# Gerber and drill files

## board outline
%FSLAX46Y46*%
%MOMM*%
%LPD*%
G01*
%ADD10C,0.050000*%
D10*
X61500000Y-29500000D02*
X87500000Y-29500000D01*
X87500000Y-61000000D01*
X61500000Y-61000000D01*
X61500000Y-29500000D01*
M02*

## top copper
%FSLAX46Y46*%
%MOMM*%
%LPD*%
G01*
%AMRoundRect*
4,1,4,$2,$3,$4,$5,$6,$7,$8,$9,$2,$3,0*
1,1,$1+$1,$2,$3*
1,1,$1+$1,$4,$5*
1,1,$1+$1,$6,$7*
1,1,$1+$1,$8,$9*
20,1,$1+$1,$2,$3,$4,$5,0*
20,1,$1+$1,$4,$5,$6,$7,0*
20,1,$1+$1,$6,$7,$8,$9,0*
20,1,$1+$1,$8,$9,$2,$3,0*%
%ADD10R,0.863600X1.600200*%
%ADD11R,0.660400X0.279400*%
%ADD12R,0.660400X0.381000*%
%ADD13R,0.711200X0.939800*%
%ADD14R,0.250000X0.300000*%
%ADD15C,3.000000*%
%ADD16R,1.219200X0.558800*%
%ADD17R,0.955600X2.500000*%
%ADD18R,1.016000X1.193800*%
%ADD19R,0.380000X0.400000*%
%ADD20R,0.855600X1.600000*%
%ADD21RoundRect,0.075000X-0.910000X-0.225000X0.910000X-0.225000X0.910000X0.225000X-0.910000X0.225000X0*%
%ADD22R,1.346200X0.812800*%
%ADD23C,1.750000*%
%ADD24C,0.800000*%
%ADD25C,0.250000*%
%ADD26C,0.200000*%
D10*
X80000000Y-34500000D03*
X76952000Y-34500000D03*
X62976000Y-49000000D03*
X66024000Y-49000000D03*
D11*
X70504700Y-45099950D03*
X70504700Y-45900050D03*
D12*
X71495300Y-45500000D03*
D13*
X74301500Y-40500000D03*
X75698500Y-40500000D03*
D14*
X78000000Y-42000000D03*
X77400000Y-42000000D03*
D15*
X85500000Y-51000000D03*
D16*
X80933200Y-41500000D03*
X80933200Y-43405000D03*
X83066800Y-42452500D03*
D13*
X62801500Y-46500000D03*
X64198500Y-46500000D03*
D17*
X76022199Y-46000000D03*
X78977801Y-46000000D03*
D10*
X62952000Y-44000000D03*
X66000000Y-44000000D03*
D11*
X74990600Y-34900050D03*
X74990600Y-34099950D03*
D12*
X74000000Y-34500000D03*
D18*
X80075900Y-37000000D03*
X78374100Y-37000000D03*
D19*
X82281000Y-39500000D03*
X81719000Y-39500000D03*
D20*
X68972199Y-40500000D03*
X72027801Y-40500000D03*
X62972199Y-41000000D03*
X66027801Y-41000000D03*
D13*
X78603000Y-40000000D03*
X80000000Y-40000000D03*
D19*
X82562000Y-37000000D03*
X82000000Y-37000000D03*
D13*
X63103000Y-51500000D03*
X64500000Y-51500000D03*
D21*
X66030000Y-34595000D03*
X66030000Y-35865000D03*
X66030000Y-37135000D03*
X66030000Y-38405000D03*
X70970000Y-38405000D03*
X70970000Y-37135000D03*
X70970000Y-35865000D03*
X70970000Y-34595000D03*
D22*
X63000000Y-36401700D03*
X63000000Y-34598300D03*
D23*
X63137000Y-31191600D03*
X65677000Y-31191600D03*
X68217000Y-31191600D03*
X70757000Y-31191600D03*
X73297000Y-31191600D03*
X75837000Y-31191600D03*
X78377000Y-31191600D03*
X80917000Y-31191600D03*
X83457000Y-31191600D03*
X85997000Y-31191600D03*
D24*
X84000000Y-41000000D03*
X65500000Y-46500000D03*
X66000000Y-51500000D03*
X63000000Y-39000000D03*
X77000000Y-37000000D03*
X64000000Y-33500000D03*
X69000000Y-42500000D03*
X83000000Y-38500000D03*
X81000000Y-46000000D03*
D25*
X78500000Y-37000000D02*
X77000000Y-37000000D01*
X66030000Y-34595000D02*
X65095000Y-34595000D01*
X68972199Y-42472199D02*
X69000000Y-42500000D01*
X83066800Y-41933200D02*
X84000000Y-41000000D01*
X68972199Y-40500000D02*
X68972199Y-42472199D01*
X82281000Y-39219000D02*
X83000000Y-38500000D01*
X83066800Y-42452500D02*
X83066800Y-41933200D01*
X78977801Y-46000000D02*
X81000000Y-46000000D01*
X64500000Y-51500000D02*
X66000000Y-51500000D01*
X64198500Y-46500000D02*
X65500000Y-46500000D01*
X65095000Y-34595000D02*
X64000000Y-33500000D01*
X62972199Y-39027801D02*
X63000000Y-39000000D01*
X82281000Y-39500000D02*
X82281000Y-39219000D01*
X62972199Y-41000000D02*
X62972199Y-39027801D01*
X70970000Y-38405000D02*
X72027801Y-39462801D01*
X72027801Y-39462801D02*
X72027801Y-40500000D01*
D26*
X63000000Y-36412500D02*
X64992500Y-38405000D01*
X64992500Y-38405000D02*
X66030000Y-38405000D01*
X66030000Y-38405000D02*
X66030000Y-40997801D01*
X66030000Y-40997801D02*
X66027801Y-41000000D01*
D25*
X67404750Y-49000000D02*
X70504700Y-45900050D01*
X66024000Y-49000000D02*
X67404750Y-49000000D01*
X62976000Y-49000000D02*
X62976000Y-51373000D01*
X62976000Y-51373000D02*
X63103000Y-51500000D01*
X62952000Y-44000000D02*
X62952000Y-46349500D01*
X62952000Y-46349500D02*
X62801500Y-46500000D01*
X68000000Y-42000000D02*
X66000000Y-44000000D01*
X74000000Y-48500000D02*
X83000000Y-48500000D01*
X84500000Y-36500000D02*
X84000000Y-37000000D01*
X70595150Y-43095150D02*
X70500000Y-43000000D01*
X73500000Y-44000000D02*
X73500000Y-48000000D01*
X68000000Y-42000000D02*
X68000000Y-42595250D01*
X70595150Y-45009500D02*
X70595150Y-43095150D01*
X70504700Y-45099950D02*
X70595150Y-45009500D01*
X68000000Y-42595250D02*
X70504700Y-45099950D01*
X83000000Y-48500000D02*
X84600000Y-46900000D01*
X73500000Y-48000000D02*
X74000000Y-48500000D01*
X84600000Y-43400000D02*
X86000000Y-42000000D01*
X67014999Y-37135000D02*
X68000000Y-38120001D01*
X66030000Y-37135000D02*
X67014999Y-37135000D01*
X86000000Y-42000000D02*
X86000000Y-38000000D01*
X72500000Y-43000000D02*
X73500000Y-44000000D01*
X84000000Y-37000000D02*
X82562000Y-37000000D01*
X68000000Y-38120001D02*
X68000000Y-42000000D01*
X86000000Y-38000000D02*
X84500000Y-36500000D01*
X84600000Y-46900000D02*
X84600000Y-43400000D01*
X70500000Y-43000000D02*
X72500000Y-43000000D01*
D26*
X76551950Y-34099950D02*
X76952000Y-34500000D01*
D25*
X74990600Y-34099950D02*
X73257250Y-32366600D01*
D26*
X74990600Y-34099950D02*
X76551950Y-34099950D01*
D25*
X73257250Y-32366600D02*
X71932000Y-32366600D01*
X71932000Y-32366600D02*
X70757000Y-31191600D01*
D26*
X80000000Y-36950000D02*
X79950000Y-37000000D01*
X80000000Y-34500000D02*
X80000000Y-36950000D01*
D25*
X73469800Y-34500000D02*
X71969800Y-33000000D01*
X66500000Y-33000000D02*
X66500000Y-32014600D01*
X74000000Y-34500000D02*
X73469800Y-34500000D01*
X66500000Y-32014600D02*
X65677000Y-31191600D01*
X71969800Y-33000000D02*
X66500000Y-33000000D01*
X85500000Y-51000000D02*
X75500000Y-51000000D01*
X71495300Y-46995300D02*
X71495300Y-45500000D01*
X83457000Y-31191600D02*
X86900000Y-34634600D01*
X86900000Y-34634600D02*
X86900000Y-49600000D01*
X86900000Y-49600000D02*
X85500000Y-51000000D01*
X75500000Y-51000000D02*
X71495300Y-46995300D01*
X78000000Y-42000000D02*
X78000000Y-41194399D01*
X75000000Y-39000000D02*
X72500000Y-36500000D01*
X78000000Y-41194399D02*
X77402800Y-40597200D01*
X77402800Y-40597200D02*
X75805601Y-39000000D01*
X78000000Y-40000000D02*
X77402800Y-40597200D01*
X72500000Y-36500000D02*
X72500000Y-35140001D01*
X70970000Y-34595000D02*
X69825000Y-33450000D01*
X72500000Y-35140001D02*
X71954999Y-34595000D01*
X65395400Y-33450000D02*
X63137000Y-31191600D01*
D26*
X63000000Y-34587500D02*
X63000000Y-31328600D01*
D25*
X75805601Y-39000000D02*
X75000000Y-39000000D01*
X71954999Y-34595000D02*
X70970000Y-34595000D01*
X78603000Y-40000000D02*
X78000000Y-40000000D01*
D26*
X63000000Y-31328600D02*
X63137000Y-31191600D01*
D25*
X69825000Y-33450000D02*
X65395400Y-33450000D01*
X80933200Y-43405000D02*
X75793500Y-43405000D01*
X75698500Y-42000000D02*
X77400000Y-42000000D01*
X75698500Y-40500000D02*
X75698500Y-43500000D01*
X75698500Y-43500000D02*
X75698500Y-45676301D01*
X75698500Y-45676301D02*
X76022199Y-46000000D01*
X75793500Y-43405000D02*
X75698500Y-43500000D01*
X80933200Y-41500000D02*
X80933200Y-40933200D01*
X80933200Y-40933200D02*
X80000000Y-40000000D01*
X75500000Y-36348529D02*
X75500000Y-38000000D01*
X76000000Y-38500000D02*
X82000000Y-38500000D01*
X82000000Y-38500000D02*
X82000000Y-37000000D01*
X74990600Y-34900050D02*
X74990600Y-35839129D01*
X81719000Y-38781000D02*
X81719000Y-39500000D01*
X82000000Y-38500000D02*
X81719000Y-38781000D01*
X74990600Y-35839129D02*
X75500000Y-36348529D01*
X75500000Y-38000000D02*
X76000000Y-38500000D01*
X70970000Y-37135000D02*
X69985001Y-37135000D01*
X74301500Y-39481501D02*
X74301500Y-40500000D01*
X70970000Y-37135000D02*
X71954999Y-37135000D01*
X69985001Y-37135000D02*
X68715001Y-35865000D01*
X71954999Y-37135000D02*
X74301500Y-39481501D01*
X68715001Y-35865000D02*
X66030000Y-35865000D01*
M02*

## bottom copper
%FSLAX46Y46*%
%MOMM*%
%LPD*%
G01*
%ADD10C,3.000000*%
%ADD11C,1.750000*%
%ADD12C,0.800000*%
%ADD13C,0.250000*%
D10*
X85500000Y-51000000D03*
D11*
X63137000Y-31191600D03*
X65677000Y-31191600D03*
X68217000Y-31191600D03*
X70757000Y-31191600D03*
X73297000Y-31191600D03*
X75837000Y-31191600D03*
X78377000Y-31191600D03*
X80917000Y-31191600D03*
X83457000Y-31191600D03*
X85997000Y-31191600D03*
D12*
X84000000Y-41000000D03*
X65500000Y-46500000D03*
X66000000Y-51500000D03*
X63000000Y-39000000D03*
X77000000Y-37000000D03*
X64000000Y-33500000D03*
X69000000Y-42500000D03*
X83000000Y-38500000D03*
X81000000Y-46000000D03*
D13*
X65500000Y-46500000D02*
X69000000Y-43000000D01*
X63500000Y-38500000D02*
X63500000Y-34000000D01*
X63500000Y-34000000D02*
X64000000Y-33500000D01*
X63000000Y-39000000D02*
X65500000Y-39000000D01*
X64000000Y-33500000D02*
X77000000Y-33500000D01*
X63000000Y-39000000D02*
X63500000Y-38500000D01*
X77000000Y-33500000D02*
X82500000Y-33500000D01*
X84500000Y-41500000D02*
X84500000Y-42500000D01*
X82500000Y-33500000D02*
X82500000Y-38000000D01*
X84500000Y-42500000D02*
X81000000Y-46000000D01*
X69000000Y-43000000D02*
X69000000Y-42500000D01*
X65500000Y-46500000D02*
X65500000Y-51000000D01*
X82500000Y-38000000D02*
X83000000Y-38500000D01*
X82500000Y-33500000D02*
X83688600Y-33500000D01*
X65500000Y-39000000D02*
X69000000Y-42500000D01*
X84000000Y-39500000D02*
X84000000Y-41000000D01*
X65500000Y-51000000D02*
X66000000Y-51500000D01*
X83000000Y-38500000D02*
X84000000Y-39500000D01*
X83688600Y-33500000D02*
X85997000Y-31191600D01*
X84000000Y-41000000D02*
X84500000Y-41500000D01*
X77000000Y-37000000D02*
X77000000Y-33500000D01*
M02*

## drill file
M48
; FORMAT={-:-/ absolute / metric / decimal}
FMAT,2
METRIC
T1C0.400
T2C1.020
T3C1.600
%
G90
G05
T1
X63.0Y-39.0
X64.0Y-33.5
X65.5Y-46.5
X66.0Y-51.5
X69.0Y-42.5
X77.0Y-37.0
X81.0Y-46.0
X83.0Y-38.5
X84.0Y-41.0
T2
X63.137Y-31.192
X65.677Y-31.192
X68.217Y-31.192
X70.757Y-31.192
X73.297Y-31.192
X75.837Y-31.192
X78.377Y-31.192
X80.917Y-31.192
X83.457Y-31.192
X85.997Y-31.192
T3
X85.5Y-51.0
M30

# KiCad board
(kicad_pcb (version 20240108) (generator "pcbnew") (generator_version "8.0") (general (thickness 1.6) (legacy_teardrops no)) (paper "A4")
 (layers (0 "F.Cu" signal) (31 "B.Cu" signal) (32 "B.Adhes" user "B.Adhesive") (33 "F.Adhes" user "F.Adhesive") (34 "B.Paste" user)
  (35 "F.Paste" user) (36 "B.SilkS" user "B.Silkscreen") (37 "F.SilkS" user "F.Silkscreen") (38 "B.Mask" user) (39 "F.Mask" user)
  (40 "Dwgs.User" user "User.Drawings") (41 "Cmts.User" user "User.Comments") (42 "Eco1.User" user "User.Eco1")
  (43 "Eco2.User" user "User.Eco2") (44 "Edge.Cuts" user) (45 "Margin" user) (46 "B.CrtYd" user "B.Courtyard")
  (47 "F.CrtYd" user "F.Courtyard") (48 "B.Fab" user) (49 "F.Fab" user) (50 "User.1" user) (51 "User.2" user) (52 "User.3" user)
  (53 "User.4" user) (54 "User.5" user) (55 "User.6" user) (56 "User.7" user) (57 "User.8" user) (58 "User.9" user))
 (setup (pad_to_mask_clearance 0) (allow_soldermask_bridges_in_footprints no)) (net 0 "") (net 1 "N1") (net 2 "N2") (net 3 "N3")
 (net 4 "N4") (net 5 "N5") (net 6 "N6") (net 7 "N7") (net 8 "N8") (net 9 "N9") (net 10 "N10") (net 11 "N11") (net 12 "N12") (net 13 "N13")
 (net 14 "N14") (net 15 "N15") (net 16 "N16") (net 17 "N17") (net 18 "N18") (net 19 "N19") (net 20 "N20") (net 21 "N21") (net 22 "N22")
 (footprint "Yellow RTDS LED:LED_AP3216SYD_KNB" (layer "F.Cu") (at 78.476 34.5 180)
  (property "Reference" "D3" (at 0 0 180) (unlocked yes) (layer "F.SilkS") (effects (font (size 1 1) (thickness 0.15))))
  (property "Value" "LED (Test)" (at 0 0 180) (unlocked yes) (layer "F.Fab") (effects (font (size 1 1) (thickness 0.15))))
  (pad "1" smd rect (at -1.524 0 180) (size 0.8636 1.6002) (layers "F.Cu" "F.Paste" "F.Mask") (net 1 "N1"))
  (pad "2" smd rect (at 1.524 0 180) (size 0.8636 1.6002) (layers "F.Cu" "F.Paste" "F.Mask") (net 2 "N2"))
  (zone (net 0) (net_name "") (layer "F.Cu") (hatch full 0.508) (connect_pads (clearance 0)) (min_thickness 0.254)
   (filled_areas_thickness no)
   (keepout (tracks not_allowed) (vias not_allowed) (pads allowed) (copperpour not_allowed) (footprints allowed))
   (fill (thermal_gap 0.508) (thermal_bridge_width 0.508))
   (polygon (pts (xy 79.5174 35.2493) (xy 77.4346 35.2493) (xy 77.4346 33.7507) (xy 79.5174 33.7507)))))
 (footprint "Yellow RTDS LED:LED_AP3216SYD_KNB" (layer "F.Cu") (at 64.5 49)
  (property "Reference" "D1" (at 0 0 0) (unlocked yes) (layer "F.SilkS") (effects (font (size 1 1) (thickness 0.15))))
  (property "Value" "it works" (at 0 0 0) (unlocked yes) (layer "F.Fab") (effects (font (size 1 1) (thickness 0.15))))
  (pad "1" smd rect (at -1.524 0) (size 0.8636 1.6002) (layers "F.Cu" "F.Paste" "F.Mask") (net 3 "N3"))
  (pad "2" smd rect (at 1.524 0) (size 0.8636 1.6002) (layers "F.Cu" "F.Paste" "F.Mask") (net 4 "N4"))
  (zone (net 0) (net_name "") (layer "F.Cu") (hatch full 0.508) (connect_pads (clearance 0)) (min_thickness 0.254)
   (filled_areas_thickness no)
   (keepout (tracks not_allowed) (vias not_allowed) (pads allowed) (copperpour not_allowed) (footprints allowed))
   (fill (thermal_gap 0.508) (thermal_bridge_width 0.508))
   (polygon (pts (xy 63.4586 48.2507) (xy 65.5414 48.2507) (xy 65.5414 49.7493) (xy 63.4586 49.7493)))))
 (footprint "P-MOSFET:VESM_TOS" (layer "F.Cu") (at 71 45.5 -90)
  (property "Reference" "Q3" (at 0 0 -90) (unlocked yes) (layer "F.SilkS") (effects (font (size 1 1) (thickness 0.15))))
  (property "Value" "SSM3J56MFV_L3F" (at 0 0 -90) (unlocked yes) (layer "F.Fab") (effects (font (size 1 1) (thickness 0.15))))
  (pad "1" smd rect (at -0.40005 0.4953 270) (size 0.2794 0.6604) (layers "F.Cu" "F.Paste" "F.Mask") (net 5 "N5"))
  (pad "2" smd rect (at 0.40005 0.4953 270) (size 0.2794 0.6604) (layers "F.Cu" "F.Paste" "F.Mask") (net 4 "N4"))
  (pad "3" smd rect (at 0 -0.4953 270) (size 0.381 0.6604) (layers "F.Cu" "F.Paste" "F.Mask") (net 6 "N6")))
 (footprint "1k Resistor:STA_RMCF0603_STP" (layer "F.Cu") (at 75 40.5)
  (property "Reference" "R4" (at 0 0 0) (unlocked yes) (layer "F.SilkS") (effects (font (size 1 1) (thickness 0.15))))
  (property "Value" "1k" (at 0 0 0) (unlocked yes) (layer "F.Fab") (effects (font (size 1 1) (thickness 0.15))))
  (pad "1" smd rect (at -0.6985 0) (size 0.7112 0.9398) (layers "F.Cu" "F.Paste" "F.Mask") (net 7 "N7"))
  (pad "2" smd rect (at 0.6985 0) (size 0.7112 0.9398) (layers "F.Cu" "F.Paste" "F.Mask") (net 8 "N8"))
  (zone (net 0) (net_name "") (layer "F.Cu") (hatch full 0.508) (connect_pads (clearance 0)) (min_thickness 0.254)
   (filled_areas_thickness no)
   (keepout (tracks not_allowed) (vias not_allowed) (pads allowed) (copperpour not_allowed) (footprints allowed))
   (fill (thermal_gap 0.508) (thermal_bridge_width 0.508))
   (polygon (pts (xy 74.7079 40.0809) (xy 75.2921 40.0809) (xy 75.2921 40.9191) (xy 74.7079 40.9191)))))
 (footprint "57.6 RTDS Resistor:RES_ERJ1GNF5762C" (layer "F.Cu") (at 77.7 42 180)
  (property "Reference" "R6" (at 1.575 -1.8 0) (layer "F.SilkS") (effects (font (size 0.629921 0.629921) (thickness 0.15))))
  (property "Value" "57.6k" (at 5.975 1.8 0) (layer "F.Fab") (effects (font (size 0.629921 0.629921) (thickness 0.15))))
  (pad "1" smd rect (at -0.3 0 180) (size 0.25 0.3) (layers "F.Cu" "F.Paste" "F.Mask") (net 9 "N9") (solder_mask_margin 0.102))
  (pad "2" smd rect (at 0.3 0 180) (size 0.25 0.3) (layers "F.Cu" "F.Paste" "F.Mask") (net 8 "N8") (solder_mask_margin 0.102)))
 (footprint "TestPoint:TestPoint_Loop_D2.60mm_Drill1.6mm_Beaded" (layer "F.Cu") (at 85.5 51)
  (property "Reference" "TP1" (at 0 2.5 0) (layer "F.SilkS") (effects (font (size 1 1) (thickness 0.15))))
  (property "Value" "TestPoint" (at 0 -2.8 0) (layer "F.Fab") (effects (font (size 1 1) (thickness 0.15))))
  (pad "1" thru_hole circle (at 0 0) (size 3 3) (drill 1.6) (layers "*.Cu" "*.Mask") (remove_unused_layers no) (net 6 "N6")))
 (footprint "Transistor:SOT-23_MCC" (layer "F.Cu") (at 82 42.4525 -90)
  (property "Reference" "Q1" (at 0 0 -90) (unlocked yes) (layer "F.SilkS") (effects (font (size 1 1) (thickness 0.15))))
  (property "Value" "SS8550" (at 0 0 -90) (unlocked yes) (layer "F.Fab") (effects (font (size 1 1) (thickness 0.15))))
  (pad "1" smd rect (at -0.9525 1.0668 270) (size 0.5588 1.2192) (layers "F.Cu" "F.Paste" "F.Mask") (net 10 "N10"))
  (pad "2" smd rect (at 0.9525 1.0668 270) (size 0.5588 1.2192) (layers "F.Cu" "F.Paste" "F.Mask") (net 8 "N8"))
  (pad "3" smd rect (at 0 -1.0668 270) (size 0.5588 1.2192) (layers "F.Cu" "F.Paste" "F.Mask") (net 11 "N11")))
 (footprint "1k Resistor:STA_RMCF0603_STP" (layer "F.Cu") (at 63.5 46.5)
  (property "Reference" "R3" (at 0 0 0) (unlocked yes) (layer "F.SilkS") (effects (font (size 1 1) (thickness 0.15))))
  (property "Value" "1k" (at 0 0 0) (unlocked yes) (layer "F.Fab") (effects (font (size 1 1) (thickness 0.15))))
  (pad "1" smd rect (at -0.6985 0) (size 0.7112 0.9398) (layers "F.Cu" "F.Paste" "F.Mask") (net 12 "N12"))
  (pad "2" smd rect (at 0.6985 0) (size 0.7112 0.9398) (layers "F.Cu" "F.Paste" "F.Mask") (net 11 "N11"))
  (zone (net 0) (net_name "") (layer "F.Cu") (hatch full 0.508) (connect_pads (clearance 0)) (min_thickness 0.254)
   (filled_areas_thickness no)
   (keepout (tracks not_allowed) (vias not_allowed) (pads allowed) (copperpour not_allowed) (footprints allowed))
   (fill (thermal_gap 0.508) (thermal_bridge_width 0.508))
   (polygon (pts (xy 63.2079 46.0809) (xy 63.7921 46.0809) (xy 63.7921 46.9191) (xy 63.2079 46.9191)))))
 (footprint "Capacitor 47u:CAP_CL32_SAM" (layer "F.Cu") (at 77.5 46)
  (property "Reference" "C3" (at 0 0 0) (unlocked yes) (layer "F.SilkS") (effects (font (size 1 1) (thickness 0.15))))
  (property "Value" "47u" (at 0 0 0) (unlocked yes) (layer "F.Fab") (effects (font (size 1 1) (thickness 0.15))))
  (pad "1" smd rect (at -1.477801 0) (size 0.9556 2.5) (layers "F.Cu" "F.Paste" "F.Mask") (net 8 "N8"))
  (pad "2" smd rect (at 1.477801 0) (size 0.9556 2.5) (layers "F.Cu" "F.Paste" "F.Mask") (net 11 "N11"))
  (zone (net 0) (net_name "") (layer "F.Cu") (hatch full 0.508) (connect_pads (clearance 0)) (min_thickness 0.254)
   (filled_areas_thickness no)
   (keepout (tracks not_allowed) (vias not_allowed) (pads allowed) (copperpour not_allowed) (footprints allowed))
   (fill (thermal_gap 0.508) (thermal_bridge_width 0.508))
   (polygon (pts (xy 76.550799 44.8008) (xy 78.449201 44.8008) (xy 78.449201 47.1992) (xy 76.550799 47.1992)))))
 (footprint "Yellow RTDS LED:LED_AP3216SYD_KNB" (layer "F.Cu") (at 64.476 44)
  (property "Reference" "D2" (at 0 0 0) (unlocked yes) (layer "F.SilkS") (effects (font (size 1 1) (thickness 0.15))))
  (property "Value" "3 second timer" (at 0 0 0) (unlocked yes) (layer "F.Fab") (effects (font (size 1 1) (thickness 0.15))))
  (pad "1" smd rect (at -1.524 0) (size 0.8636 1.6002) (layers "F.Cu" "F.Paste" "F.Mask") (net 12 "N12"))
  (pad "2" smd rect (at 1.524 0) (size 0.8636 1.6002) (layers "F.Cu" "F.Paste" "F.Mask") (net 5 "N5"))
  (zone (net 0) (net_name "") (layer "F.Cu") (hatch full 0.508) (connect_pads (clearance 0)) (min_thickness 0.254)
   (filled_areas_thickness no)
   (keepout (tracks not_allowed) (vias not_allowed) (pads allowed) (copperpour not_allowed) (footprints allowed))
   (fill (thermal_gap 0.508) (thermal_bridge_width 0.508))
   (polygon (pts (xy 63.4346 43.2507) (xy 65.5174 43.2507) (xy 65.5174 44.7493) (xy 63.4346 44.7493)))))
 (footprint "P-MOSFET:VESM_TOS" (layer "F.Cu") (at 74.4953 34.5 90)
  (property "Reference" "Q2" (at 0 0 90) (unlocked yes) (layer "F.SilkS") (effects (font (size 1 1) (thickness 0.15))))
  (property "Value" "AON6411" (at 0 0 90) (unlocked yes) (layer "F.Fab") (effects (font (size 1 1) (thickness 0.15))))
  (pad "1" smd rect (at -0.40005 0.4953 90) (size 0.2794 0.6604) (layers "F.Cu" "F.Paste" "F.Mask") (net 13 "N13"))
  (pad "2" smd rect (at 0.40005 0.4953 90) (size 0.2794 0.6604) (layers "F.Cu" "F.Paste" "F.Mask") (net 2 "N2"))
  (pad "3" smd rect (at 0 -0.4953 90) (size 0.381 0.6604) (layers "F.Cu" "F.Paste" "F.Mask") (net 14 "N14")))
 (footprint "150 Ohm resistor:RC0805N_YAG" (layer "F.Cu") (at 79.225 37 180)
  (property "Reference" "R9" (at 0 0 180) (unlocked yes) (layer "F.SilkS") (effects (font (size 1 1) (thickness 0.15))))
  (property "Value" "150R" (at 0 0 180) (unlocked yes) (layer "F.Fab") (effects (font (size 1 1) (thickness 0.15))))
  (pad "1" smd rect (at -0.8509 0 180) (size 1.016 1.1938) (layers "F.Cu" "F.Paste" "F.Mask") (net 1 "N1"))
  (pad "2" smd rect (at 0.8509 0 180) (size 1.016 1.1938) (layers "F.Cu" "F.Paste" "F.Mask") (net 11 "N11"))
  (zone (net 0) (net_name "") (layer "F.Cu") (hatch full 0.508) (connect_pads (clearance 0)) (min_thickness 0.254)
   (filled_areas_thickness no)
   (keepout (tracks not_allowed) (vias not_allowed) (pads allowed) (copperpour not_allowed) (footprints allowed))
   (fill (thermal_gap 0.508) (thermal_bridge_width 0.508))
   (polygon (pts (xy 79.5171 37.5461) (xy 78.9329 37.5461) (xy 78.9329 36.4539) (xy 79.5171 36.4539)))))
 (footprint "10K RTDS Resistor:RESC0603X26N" (layer "F.Cu") (at 82 39.5 180)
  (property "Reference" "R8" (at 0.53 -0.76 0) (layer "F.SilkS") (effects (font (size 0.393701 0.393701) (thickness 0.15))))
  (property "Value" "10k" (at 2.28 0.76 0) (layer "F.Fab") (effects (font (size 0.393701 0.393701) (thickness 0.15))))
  (pad "1" smd rect (at -0.281 0 180) (size 0.38 0.4) (layers "F.Cu" "F.Paste" "F.Mask") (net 11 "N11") (solder_mask_margin 0.102))
  (pad "2" smd rect (at 0.281 0 180) (size 0.38 0.4) (layers "F.Cu" "F.Paste" "F.Mask") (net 13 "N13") (solder_mask_margin 0.102)))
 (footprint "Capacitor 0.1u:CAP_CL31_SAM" (layer "F.Cu") (at 70.5 40.5)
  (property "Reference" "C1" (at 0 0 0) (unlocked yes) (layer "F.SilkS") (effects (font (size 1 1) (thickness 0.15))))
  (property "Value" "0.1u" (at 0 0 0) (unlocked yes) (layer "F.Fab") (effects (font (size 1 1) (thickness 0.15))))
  (pad "1" smd rect (at -1.527801 0) (size 0.8556 1.6) (layers "F.Cu" "F.Paste" "F.Mask") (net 11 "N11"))
  (pad "2" smd rect (at 1.527801 0) (size 0.8556 1.6) (layers "F.Cu" "F.Paste" "F.Mask") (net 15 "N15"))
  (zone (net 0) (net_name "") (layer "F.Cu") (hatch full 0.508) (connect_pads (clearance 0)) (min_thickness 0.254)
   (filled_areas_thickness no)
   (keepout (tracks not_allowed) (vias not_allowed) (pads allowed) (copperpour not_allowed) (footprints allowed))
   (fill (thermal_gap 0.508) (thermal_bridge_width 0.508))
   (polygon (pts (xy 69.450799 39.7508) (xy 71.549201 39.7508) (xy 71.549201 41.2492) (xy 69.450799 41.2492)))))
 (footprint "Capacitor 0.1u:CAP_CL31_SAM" (layer "F.Cu") (at 64.5 41)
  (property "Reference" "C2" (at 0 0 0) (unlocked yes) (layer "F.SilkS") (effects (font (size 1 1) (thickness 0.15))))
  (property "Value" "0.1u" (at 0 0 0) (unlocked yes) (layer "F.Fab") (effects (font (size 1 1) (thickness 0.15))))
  (pad "1" smd rect (at -1.527801 0) (size 0.8556 1.6) (layers "F.Cu" "F.Paste" "F.Mask") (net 11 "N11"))
  (pad "2" smd rect (at 1.527801 0) (size 0.8556 1.6) (layers "F.Cu" "F.Paste" "F.Mask") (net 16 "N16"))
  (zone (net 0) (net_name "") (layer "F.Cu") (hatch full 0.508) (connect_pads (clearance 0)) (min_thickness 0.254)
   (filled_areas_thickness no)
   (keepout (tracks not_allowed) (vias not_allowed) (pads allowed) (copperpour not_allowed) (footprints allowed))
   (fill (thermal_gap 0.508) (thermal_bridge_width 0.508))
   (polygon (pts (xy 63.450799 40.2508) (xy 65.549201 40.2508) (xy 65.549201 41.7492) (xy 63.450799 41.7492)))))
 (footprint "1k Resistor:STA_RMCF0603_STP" (layer "F.Cu") (at 79.3015 40)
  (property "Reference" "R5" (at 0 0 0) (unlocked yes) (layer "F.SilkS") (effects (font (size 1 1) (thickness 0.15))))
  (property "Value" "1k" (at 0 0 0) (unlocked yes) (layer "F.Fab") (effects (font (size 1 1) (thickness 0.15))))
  (pad "1" smd rect (at -0.6985 0) (size 0.7112 0.9398) (layers "F.Cu" "F.Paste" "F.Mask") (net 9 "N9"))
  (pad "2" smd rect (at 0.6985 0) (size 0.7112 0.9398) (layers "F.Cu" "F.Paste" "F.Mask") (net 10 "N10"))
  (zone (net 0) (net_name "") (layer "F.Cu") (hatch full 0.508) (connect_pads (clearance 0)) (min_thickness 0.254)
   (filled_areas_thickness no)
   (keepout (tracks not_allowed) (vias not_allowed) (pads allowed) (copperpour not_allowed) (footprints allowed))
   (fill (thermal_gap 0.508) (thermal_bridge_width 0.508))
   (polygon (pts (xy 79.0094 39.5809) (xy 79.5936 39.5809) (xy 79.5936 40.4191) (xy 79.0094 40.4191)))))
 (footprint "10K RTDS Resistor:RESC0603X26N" (layer "F.Cu") (at 82.281 37 180)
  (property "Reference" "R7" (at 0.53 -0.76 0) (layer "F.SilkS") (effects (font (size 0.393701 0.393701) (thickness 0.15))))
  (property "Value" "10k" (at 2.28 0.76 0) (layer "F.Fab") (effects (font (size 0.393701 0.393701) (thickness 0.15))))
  (pad "1" smd rect (at -0.281 0 180) (size 0.38 0.4) (layers "F.Cu" "F.Paste" "F.Mask") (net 5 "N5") (solder_mask_margin 0.102))
  (pad "2" smd rect (at 0.281 0 180) (size 0.38 0.4) (layers "F.Cu" "F.Paste" "F.Mask") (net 13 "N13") (solder_mask_margin 0.102)))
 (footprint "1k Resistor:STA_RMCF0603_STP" (layer "F.Cu") (at 63.8015 51.5)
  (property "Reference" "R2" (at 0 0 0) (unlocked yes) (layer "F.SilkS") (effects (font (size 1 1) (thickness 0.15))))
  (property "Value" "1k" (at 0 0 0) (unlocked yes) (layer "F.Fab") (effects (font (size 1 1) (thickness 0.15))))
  (pad "1" smd rect (at -0.6985 0) (size 0.7112 0.9398) (layers "F.Cu" "F.Paste" "F.Mask") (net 3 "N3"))
  (pad "2" smd rect (at 0.6985 0) (size 0.7112 0.9398) (layers "F.Cu" "F.Paste" "F.Mask") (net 11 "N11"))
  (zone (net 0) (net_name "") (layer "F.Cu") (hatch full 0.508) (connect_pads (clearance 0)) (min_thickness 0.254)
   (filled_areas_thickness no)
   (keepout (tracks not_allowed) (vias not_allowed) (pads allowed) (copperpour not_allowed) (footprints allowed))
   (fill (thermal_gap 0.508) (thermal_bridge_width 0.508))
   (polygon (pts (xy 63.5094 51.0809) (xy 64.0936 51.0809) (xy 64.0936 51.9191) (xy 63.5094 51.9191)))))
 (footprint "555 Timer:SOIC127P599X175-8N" (layer "F.Cu") (at 68.5 36.5)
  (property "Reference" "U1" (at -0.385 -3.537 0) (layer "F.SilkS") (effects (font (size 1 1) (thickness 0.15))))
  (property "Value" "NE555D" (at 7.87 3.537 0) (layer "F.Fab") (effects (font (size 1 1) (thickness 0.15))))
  (pad "1" smd roundrect (at -2.47 -1.905) (size 1.97 0.6) (layers "F.Cu" "F.Paste" "F.Mask") (roundrect_rratio 0.125) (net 11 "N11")
   (solder_mask_margin 0.102))
  (pad "2" smd roundrect (at -2.47 -0.635) (size 1.97 0.6) (layers "F.Cu" "F.Paste" "F.Mask") (roundrect_rratio 0.125) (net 7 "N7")
   (solder_mask_margin 0.102))
  (pad "3" smd roundrect (at -2.47 0.635) (size 1.97 0.6) (layers "F.Cu" "F.Paste" "F.Mask") (roundrect_rratio 0.125) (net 5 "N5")
   (solder_mask_margin 0.102))
  (pad "4" smd roundrect (at -2.47 1.905) (size 1.97 0.6) (layers "F.Cu" "F.Paste" "F.Mask") (roundrect_rratio 0.125) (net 16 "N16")
   (solder_mask_margin 0.102))
  (pad "5" smd roundrect (at 2.47 1.905) (size 1.97 0.6) (layers "F.Cu" "F.Paste" "F.Mask") (roundrect_rratio 0.125) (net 15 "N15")
   (solder_mask_margin 0.102))
  (pad "6" smd roundrect (at 2.47 0.635) (size 1.97 0.6) (layers "F.Cu" "F.Paste" "F.Mask") (roundrect_rratio 0.125) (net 7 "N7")
   (solder_mask_margin 0.102))
  (pad "7" smd roundrect (at 2.47 -0.635) (size 1.97 0.6) (layers "F.Cu" "F.Paste" "F.Mask") (roundrect_rratio 0.125) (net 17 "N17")
   (solder_mask_margin 0.102))
  (pad "8" smd roundrect (at 2.47 -1.905) (size 1.97 0.6) (layers "F.Cu" "F.Paste" "F.Mask") (roundrect_rratio 0.125) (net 9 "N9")
   (solder_mask_margin 0.102)))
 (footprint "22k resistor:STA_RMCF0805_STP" (layer "F.Cu") (at 63 35.5 90)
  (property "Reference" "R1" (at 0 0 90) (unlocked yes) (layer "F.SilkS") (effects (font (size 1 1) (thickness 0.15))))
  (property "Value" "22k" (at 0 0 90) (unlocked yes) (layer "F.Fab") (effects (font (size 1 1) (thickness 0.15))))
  (pad "1" smd rect (at -0.9017 0 90) (size 0.8128 1.3462) (layers "F.Cu" "F.Paste" "F.Mask") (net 16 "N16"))
  (pad "2" smd rect (at 0.9017 0 90) (size 0.8128 1.3462) (layers "F.Cu" "F.Paste" "F.Mask") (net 9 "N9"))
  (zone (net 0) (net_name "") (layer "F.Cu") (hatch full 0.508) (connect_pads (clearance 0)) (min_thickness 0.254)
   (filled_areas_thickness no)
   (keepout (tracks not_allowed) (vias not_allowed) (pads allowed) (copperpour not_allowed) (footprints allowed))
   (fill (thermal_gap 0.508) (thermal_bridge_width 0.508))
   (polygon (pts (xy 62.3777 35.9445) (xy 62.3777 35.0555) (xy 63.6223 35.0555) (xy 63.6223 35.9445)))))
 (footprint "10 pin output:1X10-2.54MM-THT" (layer "F.Cu") (at 63.137 31.1916)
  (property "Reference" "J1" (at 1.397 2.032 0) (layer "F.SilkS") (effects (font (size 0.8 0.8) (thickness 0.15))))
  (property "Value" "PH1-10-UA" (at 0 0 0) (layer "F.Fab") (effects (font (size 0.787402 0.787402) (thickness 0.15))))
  (pad "1" thru_hole circle (at 0 0) (size 1.75 1.75) (drill 1.02) (layers "*.Cu" "*.Mask") (remove_unused_layers no) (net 9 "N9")
   (solder_mask_margin 0.102))
  (pad "2" thru_hole circle (at 2.54 0) (size 1.75 1.75) (drill 1.02) (layers "*.Cu" "*.Mask") (remove_unused_layers no) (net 14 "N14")
   (solder_mask_margin 0.102))
  (pad "3" thru_hole circle (at 5.08 0) (size 1.75 1.75) (drill 1.02) (layers "*.Cu" "*.Mask") (remove_unused_layers no) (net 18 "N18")
   (solder_mask_margin 0.102))
  (pad "4" thru_hole circle (at 7.62 0) (size 1.75 1.75) (drill 1.02) (layers "*.Cu" "*.Mask") (remove_unused_layers no) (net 2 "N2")
   (solder_mask_margin 0.102))
  (pad "5" thru_hole circle (at 10.16 0) (size 1.75 1.75) (drill 1.02) (layers "*.Cu" "*.Mask") (remove_unused_layers no) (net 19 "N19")
   (solder_mask_margin 0.102))
  (pad "6" thru_hole circle (at 12.7 0) (size 1.75 1.75) (drill 1.02) (layers "*.Cu" "*.Mask") (remove_unused_layers no) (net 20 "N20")
   (solder_mask_margin 0.102))
  (pad "7" thru_hole circle (at 15.24 0) (size 1.75 1.75) (drill 1.02) (layers "*.Cu" "*.Mask") (remove_unused_layers no) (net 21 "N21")
   (solder_mask_margin 0.102))
  (pad "8" thru_hole circle (at 17.78 0) (size 1.75 1.75) (drill 1.02) (layers "*.Cu" "*.Mask") (remove_unused_layers no) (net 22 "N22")
   (solder_mask_margin 0.102))
  (pad "9" thru_hole circle (at 20.32 0) (size 1.75 1.75) (drill 1.02) (layers "*.Cu" "*.Mask") (remove_unused_layers no) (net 6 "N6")
   (solder_mask_margin 0.102))
  (pad "10" thru_hole circle (at 22.86 0) (size 1.75 1.75) (drill 1.02) (layers "*.Cu" "*.Mask") (remove_unused_layers no) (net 11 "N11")
   (solder_mask_margin 0.102)))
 (gr_rect (start 61.5 29.5) (end 87.5 61) (stroke (width 0.05) (type default)) (fill none) (layer "Edge.Cuts"))
 (segment (start 78.5 37) (end 77 37) (width 0.25) (layer "F.Cu") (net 11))
 (segment (start 66.03 34.595) (end 65.095 34.595) (width 0.25) (layer "F.Cu") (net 11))
 (segment (start 68.972199 42.472199) (end 69 42.5) (width 0.25) (layer "F.Cu") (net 11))
 (segment (start 83.0668 41.9332) (end 84 41) (width 0.25) (layer "F.Cu") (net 11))
 (segment (start 68.972199 40.5) (end 68.972199 42.472199) (width 0.25) (layer "F.Cu") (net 11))
 (segment (start 82.281 39.219) (end 83 38.5) (width 0.25) (layer "F.Cu") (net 11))
 (segment (start 83.0668 42.4525) (end 83.0668 41.9332) (width 0.25) (layer "F.Cu") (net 11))
 (segment (start 78.977801 46) (end 81 46) (width 0.25) (layer "F.Cu") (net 11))
 (segment (start 64.5 51.5) (end 66 51.5) (width 0.25) (layer "F.Cu") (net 11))
 (segment (start 64.1985 46.5) (end 65.5 46.5) (width 0.25) (layer "F.Cu") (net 11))
 (segment (start 65.095 34.595) (end 64 33.5) (width 0.25) (layer "F.Cu") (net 11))
 (segment (start 62.972199 39.027801) (end 63 39) (width 0.25) (layer "F.Cu") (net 11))
 (segment (start 82.281 39.5) (end 82.281 39.219) (width 0.25) (layer "F.Cu") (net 11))
 (segment (start 62.972199 41) (end 62.972199 39.027801) (width 0.25) (layer "F.Cu") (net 11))
 (via (at 84 41) (size 0.8) (drill 0.4) (layers "F.Cu" "B.Cu") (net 11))
 (via (at 65.5 46.5) (size 0.8) (drill 0.4) (layers "F.Cu" "B.Cu") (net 11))
 (via (at 66 51.5) (size 0.8) (drill 0.4) (layers "F.Cu" "B.Cu") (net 11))
 (via (at 63 39) (size 0.8) (drill 0.4) (layers "F.Cu" "B.Cu") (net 11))
 (via (at 77 37) (size 0.8) (drill 0.4) (layers "F.Cu" "B.Cu") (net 11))
 (via (at 64 33.5) (size 0.8) (drill 0.4) (layers "F.Cu" "B.Cu") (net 11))
 (via (at 69 42.5) (size 0.8) (drill 0.4) (layers "F.Cu" "B.Cu") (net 11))
 (via (at 83 38.5) (size 0.8) (drill 0.4) (layers "F.Cu" "B.Cu") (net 11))
 (via (at 81 46) (size 0.8) (drill 0.4) (layers "F.Cu" "B.Cu") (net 11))
 (segment (start 65.5 46.5) (end 69 43) (width 0.25) (layer "B.Cu") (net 11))
 (segment (start 63.5 38.5) (end 63.5 34) (width 0.25) (layer "B.Cu") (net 11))
 (segment (start 63.5 34) (end 64 33.5) (width 0.25) (layer "B.Cu") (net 11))
 (segment (start 63 39) (end 65.5 39) (width 0.25) (layer "B.Cu") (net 11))
 (segment (start 64 33.5) (end 77 33.5) (width 0.25) (layer "B.Cu") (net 11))
 (segment (start 63 39) (end 63.5 38.5) (width 0.25) (layer "B.Cu") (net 11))
 (segment (start 77 33.5) (end 82.5 33.5) (width 0.25) (layer "B.Cu") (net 11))
 (segment (start 84.5 41.5) (end 84.5 42.5) (width 0.25) (layer "B.Cu") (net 11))
 (segment (start 82.5 33.5) (end 82.5 38) (width 0.25) (layer "B.Cu") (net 11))
 (segment (start 84.5 42.5) (end 81 46) (width 0.25) (layer "B.Cu") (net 11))
 (segment (start 69 43) (end 69 42.5) (width 0.25) (layer "B.Cu") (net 11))
 (segment (start 65.5 46.5) (end 65.5 51) (width 0.25) (layer "B.Cu") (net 11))
 (segment (start 82.5 38) (end 83 38.5) (width 0.25) (layer "B.Cu") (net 11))
 (segment (start 82.5 33.5) (end 83.6886 33.5) (width 0.25) (layer "B.Cu") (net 11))
 (segment (start 65.5 39) (end 69 42.5) (width 0.25) (layer "B.Cu") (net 11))
 (segment (start 84 39.5) (end 84 41) (width 0.25) (layer "B.Cu") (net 11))
 (segment (start 65.5 51) (end 66 51.5) (width 0.25) (layer "B.Cu") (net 11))
 (segment (start 83 38.5) (end 84 39.5) (width 0.25) (layer "B.Cu") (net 11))
 (segment (start 83.6886 33.5) (end 85.997 31.1916) (width 0.25) (layer "B.Cu") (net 11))
 (segment (start 84 41) (end 84.5 41.5) (width 0.25) (layer "B.Cu") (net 11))
 (segment (start 77 37) (end 77 33.5) (width 0.25) (layer "B.Cu") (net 11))
 (segment (start 70.97 38.405) (end 72.027801 39.462801) (width 0.25) (layer "F.Cu") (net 15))
 (segment (start 72.027801 39.462801) (end 72.027801 40.5) (width 0.25) (layer "F.Cu") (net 15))
 (segment (start 63 36.4125) (end 64.9925 38.405) (width 0.2) (layer "F.Cu") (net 16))
 (segment (start 64.9925 38.405) (end 66.03 38.405) (width 0.2) (layer "F.Cu") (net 16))
 (segment (start 66.03 38.405) (end 66.03 40.997801) (width 0.2) (layer "F.Cu") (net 16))
 (segment (start 66.03 40.997801) (end 66.027801 41) (width 0.2) (layer "F.Cu") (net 16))
 (segment (start 67.40475 49) (end 70.5047 45.90005) (width 0.25) (layer "F.Cu") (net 4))
 (segment (start 66.024 49) (end 67.40475 49) (width 0.25) (layer "F.Cu") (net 4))
 (segment (start 62.976 49) (end 62.976 51.373) (width 0.25) (layer "F.Cu") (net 3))
 (segment (start 62.976 51.373) (end 63.103 51.5) (width 0.25) (layer "F.Cu") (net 3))
 (segment (start 62.952 44) (end 62.952 46.3495) (width 0.25) (layer "F.Cu") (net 12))
 (segment (start 62.952 46.3495) (end 62.8015 46.5) (width 0.25) (layer "F.Cu") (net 12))
 (segment (start 68 42) (end 66 44) (width 0.25) (layer "F.Cu") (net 5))
 (segment (start 74 48.5) (end 83 48.5) (width 0.25) (layer "F.Cu") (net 5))
 (segment (start 84.5 36.5) (end 84 37) (width 0.25) (layer "F.Cu") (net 5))
 (segment (start 70.59515 43.09515) (end 70.5 43) (width 0.25) (layer "F.Cu") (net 5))
 (segment (start 73.5 44) (end 73.5 48) (width 0.25) (layer "F.Cu") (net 5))
 (segment (start 68 42) (end 68 42.59525) (width 0.25) (layer "F.Cu") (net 5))
 (segment (start 70.59515 45.0095) (end 70.59515 43.09515) (width 0.25) (layer "F.Cu") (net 5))
 (segment (start 70.5047 45.09995) (end 70.59515 45.0095) (width 0.25) (layer "F.Cu") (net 5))
 (segment (start 68 42.59525) (end 70.5047 45.09995) (width 0.25) (layer "F.Cu") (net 5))
 (segment (start 83 48.5) (end 84.6 46.9) (width 0.25) (layer "F.Cu") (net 5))
 (segment (start 73.5 48) (end 74 48.5) (width 0.25) (layer "F.Cu") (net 5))
 (segment (start 84.6 43.4) (end 86 42) (width 0.25) (layer "F.Cu") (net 5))
 (segment (start 67.014999 37.135) (end 68 38.120001) (width 0.25) (layer "F.Cu") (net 5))
 (segment (start 66.03 37.135) (end 67.014999 37.135) (width 0.25) (layer "F.Cu") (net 5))
 (segment (start 86 42) (end 86 38) (width 0.25) (layer "F.Cu") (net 5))
 (segment (start 72.5 43) (end 73.5 44) (width 0.25) (layer "F.Cu") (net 5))
 (segment (start 84 37) (end 82.562 37) (width 0.25) (layer "F.Cu") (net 5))
 (segment (start 68 38.120001) (end 68 42) (width 0.25) (layer "F.Cu") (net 5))
 (segment (start 86 38) (end 84.5 36.5) (width 0.25) (layer "F.Cu") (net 5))
 (segment (start 84.6 46.9) (end 84.6 43.4) (width 0.25) (layer "F.Cu") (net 5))
 (segment (start 70.5 43) (end 72.5 43) (width 0.25) (layer "F.Cu") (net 5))
 (segment (start 76.55195 34.09995) (end 76.952 34.5) (width 0.2) (layer "F.Cu") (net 2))
 (segment (start 74.9906 34.09995) (end 73.25725 32.3666) (width 0.25) (layer "F.Cu") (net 2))
 (segment (start 74.9906 34.09995) (end 76.55195 34.09995) (width 0.2) (layer "F.Cu") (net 2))
 (segment (start 73.25725 32.3666) (end 71.932 32.3666) (width 0.25) (layer "F.Cu") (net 2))
 (segment (start 71.932 32.3666) (end 70.757 31.1916) (width 0.25) (layer "F.Cu") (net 2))
 (segment (start 80 36.95) (end 79.95 37) (width 0.2) (layer "F.Cu") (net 1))
 (segment (start 80 34.5) (end 80 36.95) (width 0.2) (layer "F.Cu") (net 1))
 (segment (start 73.4698 34.5) (end 71.9698 33) (width 0.25) (layer "F.Cu") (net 14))
 (segment (start 66.5 33) (end 66.5 32.0146) (width 0.25) (layer "F.Cu") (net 14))
 (segment (start 74 34.5) (end 73.4698 34.5) (width 0.25) (layer "F.Cu") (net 14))
 (segment (start 66.5 32.0146) (end 65.677 31.1916) (width 0.25) (layer "F.Cu") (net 14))
 (segment (start 71.9698 33) (end 66.5 33) (width 0.25) (layer "F.Cu") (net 14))
 (segment (start 85.5 51) (end 75.5 51) (width 0.25) (layer "F.Cu") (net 6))
 (segment (start 71.4953 46.9953) (end 71.4953 45.5) (width 0.25) (layer "F.Cu") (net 6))
 (segment (start 83.457 31.1916) (end 86.9 34.6346) (width 0.25) (layer "F.Cu") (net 6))
 (segment (start 86.9 34.6346) (end 86.9 49.6) (width 0.25) (layer "F.Cu") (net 6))
 (segment (start 86.9 49.6) (end 85.5 51) (width 0.25) (layer "F.Cu") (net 6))
 (segment (start 75.5 51) (end 71.4953 46.9953) (width 0.25) (layer "F.Cu") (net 6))
 (segment (start 78 42) (end 78 41.194399) (width 0.25) (layer "F.Cu") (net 9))
 (segment (start 75 39) (end 72.5 36.5) (width 0.25) (layer "F.Cu") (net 9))
 (segment (start 78 41.194399) (end 77.4028 40.5972) (width 0.25) (layer "F.Cu") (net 9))
 (segment (start 77.4028 40.5972) (end 75.805601 39) (width 0.25) (layer "F.Cu") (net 9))
 (segment (start 78 40) (end 77.4028 40.5972) (width 0.25) (layer "F.Cu") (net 9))
 (segment (start 72.5 36.5) (end 72.5 35.140001) (width 0.25) (layer "F.Cu") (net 9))
 (segment (start 70.97 34.595) (end 69.825 33.45) (width 0.25) (layer "F.Cu") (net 9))
 (segment (start 72.5 35.140001) (end 71.954999 34.595) (width 0.25) (layer "F.Cu") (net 9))
 (segment (start 65.3954 33.45) (end 63.137 31.1916) (width 0.25) (layer "F.Cu") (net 9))
 (segment (start 63 34.5875) (end 63 31.3286) (width 0.2) (layer "F.Cu") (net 9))
 (segment (start 75.805601 39) (end 75 39) (width 0.25) (layer "F.Cu") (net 9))
 (segment (start 71.954999 34.595) (end 70.97 34.595) (width 0.25) (layer "F.Cu") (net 9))
 (segment (start 78.603 40) (end 78 40) (width 0.25) (layer "F.Cu") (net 9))
 (segment (start 63 31.3286) (end 63.137 31.1916) (width 0.2) (layer "F.Cu") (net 9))
 (segment (start 69.825 33.45) (end 65.3954 33.45) (width 0.25) (layer "F.Cu") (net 9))
 (segment (start 80.9332 43.405) (end 75.7935 43.405) (width 0.25) (layer "F.Cu") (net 8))
 (segment (start 75.6985 42) (end 77.4 42) (width 0.25) (layer "F.Cu") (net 8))
 (segment (start 75.6985 40.5) (end 75.6985 43.5) (width 0.25) (layer "F.Cu") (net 8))
 (segment (start 75.6985 43.5) (end 75.6985 45.676301) (width 0.25) (layer "F.Cu") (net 8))
 (segment (start 75.6985 45.676301) (end 76.022199 46) (width 0.25) (layer "F.Cu") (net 8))
 (segment (start 75.7935 43.405) (end 75.6985 43.5) (width 0.25) (layer "F.Cu") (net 8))
 (segment (start 80.9332 41.5) (end 80.9332 40.9332) (width 0.25) (layer "F.Cu") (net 10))
 (segment (start 80.9332 40.9332) (end 80 40) (width 0.25) (layer "F.Cu") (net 10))
 (segment (start 75.5 36.348529) (end 75.5 38) (width 0.25) (layer "F.Cu") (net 13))
 (segment (start 76 38.5) (end 82 38.5) (width 0.25) (layer "F.Cu") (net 13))
 (segment (start 82 38.5) (end 82 37) (width 0.25) (layer "F.Cu") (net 13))
 (segment (start 74.9906 34.90005) (end 74.9906 35.839129) (width 0.25) (layer "F.Cu") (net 13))
 (segment (start 81.719 38.781) (end 81.719 39.5) (width 0.25) (layer "F.Cu") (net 13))
 (segment (start 82 38.5) (end 81.719 38.781) (width 0.25) (layer "F.Cu") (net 13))
 (segment (start 74.9906 35.839129) (end 75.5 36.348529) (width 0.25) (layer "F.Cu") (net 13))
 (segment (start 75.5 38) (end 76 38.5) (width 0.25) (layer "F.Cu") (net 13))
 (segment (start 70.97 37.135) (end 69.985001 37.135) (width 0.25) (layer "F.Cu") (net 7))
 (segment (start 74.3015 39.481501) (end 74.3015 40.5) (width 0.25) (layer "F.Cu") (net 7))
 (segment (start 70.97 37.135) (end 71.954999 37.135) (width 0.25) (layer "F.Cu") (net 7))
 (segment (start 69.985001 37.135) (end 68.715001 35.865) (width 0.25) (layer "F.Cu") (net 7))
 (segment (start 71.954999 37.135) (end 74.3015 39.481501) (width 0.25) (layer "F.Cu") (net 7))
 (segment (start 68.715001 35.865) (end 66.03 35.865) (width 0.25) (layer "F.Cu") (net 7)))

